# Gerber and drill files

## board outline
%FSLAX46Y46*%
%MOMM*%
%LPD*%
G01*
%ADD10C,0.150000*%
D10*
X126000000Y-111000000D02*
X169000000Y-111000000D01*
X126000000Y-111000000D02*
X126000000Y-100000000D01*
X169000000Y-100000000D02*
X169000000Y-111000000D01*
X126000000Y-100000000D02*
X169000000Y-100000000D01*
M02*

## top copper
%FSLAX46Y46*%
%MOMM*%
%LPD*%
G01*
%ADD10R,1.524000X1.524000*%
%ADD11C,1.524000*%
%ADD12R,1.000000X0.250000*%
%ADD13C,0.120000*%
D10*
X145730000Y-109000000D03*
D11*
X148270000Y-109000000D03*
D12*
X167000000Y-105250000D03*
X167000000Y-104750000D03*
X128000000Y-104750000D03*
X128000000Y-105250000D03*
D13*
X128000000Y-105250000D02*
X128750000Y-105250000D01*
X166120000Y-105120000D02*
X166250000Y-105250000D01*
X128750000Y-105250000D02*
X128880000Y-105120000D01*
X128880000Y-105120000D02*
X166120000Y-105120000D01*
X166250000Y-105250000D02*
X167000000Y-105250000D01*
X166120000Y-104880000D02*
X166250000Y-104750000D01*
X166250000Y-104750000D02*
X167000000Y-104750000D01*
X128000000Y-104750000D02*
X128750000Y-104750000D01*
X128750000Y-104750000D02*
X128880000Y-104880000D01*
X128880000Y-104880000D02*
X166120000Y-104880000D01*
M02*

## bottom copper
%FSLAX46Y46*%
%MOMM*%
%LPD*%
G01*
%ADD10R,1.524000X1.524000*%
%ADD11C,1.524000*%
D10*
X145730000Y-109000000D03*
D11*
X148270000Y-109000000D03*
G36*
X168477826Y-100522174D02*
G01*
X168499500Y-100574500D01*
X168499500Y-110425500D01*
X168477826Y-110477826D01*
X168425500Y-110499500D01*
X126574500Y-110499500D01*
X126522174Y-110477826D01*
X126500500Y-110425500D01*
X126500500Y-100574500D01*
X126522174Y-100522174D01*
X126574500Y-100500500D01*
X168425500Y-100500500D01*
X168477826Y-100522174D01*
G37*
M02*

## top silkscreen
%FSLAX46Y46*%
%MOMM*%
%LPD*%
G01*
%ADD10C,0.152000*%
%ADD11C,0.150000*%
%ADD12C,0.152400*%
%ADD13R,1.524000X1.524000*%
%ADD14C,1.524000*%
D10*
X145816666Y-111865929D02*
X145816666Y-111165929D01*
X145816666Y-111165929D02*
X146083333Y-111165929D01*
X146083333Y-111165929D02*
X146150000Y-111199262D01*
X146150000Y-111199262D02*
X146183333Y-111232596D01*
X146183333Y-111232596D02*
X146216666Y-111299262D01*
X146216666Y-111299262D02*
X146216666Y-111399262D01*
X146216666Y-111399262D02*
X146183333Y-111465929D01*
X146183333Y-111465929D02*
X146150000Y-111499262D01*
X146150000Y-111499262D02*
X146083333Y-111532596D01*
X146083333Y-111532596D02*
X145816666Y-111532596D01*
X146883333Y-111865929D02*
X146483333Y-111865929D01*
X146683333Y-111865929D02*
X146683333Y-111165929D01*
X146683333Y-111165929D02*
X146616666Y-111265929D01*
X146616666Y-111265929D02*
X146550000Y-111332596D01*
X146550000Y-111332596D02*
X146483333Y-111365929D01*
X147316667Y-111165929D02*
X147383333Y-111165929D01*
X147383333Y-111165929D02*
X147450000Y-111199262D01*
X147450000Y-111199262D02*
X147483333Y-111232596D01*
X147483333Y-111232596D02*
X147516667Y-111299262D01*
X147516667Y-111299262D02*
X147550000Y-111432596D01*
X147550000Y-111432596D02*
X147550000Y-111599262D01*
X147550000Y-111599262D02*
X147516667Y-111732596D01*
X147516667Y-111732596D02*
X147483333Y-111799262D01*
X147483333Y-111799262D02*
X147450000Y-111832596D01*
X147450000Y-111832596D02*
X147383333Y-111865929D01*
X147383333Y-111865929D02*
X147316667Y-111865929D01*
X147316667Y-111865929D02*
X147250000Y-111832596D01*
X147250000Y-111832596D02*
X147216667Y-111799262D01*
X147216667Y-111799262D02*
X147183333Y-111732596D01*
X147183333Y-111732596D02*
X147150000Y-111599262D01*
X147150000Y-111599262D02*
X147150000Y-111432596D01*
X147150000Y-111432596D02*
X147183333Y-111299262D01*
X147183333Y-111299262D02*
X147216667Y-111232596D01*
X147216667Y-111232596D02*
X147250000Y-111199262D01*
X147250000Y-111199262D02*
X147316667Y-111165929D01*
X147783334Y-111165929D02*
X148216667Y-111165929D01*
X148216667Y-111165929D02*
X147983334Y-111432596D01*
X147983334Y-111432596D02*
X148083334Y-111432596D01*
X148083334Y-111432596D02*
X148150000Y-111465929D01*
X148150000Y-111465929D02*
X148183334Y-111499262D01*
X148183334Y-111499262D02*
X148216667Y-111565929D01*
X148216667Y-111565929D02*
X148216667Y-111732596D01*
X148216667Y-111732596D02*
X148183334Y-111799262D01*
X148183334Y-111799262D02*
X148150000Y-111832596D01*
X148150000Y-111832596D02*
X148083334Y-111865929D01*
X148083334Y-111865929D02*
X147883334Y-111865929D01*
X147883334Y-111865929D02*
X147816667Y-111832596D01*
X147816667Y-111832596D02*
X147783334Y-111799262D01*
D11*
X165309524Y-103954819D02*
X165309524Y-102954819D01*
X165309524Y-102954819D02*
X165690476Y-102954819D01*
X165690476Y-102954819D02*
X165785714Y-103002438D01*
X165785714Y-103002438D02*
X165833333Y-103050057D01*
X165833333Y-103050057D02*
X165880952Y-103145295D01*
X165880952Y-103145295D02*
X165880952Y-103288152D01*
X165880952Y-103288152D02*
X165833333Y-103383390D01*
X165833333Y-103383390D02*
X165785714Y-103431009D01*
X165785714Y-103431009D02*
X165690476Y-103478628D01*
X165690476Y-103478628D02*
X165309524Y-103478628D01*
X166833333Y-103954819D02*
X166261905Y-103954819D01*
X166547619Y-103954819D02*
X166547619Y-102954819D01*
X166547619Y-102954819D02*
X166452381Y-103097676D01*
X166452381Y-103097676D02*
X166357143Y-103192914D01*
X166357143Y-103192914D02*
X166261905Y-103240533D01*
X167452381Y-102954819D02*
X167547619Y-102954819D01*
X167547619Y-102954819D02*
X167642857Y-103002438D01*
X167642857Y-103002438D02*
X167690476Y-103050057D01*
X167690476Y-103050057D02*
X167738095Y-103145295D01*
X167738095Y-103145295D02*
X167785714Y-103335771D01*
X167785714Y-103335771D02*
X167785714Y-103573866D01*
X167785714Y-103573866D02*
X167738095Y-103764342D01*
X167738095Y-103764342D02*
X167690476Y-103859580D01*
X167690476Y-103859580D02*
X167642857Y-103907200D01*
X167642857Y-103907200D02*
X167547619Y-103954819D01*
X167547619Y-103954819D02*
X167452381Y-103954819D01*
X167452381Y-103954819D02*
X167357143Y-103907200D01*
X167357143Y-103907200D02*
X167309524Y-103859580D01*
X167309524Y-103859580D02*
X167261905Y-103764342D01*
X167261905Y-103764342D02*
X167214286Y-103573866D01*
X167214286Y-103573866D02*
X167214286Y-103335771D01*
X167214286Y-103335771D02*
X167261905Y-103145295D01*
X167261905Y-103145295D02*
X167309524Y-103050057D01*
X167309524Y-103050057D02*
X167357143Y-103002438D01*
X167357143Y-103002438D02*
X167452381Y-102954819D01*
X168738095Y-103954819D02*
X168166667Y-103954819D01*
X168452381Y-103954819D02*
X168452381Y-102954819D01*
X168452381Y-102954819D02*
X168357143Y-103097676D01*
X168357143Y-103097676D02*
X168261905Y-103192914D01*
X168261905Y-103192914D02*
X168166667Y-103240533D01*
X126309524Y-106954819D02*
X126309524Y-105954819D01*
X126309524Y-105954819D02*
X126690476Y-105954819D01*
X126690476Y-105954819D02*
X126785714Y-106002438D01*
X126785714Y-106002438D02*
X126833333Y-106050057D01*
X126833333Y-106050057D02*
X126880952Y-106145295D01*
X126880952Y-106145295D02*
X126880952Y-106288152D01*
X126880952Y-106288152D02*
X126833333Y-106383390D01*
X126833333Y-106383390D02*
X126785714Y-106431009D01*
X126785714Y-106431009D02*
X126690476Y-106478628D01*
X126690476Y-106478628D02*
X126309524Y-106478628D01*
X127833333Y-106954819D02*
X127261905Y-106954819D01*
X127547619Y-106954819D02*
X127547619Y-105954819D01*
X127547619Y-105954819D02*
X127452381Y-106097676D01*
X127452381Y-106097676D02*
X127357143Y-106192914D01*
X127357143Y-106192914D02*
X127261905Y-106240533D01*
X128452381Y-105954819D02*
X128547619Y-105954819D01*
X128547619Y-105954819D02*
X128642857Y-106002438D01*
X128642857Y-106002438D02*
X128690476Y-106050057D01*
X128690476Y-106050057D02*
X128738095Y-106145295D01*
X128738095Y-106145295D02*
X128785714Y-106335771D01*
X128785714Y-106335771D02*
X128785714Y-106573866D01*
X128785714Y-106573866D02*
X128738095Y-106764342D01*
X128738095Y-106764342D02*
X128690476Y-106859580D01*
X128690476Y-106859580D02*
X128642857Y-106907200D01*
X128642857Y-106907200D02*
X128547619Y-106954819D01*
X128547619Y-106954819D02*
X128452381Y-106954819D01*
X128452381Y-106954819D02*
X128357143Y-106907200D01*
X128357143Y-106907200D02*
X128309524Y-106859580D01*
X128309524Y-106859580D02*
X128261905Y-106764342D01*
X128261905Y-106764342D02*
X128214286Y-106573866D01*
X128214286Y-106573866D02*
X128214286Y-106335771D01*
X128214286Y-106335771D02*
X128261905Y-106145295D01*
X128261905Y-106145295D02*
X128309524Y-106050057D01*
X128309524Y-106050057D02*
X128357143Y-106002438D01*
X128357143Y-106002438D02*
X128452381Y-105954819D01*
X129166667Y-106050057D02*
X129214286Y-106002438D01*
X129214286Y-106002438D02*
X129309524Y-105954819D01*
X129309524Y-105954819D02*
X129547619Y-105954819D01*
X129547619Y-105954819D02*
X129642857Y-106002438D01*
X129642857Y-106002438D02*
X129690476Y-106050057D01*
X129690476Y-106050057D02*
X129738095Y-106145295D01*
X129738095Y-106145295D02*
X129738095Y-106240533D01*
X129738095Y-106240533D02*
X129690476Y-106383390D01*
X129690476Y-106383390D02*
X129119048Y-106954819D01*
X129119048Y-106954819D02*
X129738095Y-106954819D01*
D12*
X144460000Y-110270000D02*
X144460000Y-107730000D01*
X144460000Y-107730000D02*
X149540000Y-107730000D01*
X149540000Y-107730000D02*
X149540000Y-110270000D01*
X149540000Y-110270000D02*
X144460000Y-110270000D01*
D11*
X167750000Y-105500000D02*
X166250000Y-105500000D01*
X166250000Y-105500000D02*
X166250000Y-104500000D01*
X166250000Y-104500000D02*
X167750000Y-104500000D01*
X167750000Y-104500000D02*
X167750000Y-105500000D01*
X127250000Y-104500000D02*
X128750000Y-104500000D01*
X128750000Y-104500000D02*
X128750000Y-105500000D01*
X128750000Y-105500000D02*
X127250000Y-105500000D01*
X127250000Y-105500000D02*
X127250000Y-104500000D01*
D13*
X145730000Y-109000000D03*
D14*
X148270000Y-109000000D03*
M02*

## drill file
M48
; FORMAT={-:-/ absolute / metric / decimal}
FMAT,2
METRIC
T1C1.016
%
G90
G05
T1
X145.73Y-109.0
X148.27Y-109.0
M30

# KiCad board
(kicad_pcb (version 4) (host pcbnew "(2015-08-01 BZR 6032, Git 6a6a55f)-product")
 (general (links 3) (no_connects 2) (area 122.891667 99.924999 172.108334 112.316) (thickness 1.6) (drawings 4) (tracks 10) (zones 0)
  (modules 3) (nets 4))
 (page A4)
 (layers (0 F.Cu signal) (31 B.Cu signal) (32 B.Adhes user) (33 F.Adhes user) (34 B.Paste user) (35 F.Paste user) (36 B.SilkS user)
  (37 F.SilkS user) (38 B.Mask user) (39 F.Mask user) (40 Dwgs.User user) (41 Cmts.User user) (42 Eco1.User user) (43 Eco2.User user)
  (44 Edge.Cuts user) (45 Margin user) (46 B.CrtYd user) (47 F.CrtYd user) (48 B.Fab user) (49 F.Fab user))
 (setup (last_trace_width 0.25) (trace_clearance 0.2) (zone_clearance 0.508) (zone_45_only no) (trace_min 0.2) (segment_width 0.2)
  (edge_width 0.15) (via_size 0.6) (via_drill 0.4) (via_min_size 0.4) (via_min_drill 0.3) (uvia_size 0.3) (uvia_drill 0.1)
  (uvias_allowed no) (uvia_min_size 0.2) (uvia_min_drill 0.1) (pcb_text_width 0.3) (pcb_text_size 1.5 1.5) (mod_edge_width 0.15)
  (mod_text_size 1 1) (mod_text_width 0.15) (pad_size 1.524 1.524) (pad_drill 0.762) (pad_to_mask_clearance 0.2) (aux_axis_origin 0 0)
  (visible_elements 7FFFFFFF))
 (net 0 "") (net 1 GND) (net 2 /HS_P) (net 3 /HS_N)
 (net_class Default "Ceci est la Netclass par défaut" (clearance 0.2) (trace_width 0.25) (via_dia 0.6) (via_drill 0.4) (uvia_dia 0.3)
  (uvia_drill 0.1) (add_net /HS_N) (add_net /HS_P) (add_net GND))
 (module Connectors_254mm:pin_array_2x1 (layer F.Cu) (at 147 109)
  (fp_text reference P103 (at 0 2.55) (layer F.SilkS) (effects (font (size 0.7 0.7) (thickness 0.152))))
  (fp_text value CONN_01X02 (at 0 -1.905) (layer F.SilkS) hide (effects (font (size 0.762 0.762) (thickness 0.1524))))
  (fp_line (start -2.54 1.27) (end -2.54 -1.27) (layer F.SilkS) (width 0.1524))
  (fp_line (start -2.54 -1.27) (end 2.54 -1.27) (layer F.SilkS) (width 0.1524))
  (fp_line (start 2.54 -1.27) (end 2.54 1.27) (layer F.SilkS) (width 0.1524))
  (fp_line (start 2.54 1.27) (end -2.54 1.27) (layer F.SilkS) (width 0.1524))
  (pad 1 thru_hole rect (at -1.27 0) (size 1.524 1.524) (drill 1.016) (layers *.Cu *.Mask F.SilkS) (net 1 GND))
  (pad 2 thru_hole circle (at 1.27 0) (size 1.524 1.524) (drill 1.016) (layers *.Cu *.Mask F.SilkS) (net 1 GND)))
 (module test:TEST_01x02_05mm (layer F.Cu) (at 167 105 180)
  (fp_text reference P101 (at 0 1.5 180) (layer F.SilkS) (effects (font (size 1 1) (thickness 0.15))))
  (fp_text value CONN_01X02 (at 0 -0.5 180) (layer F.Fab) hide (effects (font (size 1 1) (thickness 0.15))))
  (fp_line (start -0.75 -0.5) (end 0.75 -0.5) (layer F.SilkS) (width 0.15))
  (fp_line (start 0.75 -0.5) (end 0.75 0.5) (layer F.SilkS) (width 0.15))
  (fp_line (start 0.75 0.5) (end -0.75 0.5) (layer F.SilkS) (width 0.15))
  (fp_line (start -0.75 0.5) (end -0.75 -0.5) (layer F.SilkS) (width 0.15))
  (pad 1 smd rect (at 0 -0.25 180) (size 1 0.25) (layers F.Cu F.Paste F.Mask) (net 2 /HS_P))
  (pad 2 smd rect (at 0 0.25 180) (size 1 0.25) (layers F.Cu F.Paste F.Mask) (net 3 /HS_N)))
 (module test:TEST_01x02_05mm (layer F.Cu) (at 128 105)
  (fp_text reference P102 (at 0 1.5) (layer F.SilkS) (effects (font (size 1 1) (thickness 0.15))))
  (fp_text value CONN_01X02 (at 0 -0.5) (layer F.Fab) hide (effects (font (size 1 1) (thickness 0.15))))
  (fp_line (start -0.75 -0.5) (end 0.75 -0.5) (layer F.SilkS) (width 0.15))
  (fp_line (start 0.75 -0.5) (end 0.75 0.5) (layer F.SilkS) (width 0.15))
  (fp_line (start 0.75 0.5) (end -0.75 0.5) (layer F.SilkS) (width 0.15))
  (fp_line (start -0.75 0.5) (end -0.75 -0.5) (layer F.SilkS) (width 0.15))
  (pad 1 smd rect (at 0 -0.25) (size 1 0.25) (layers F.Cu F.Paste F.Mask) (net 3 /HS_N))
  (pad 2 smd rect (at 0 0.25) (size 1 0.25) (layers F.Cu F.Paste F.Mask) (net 2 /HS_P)))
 (gr_line (start 126 111) (end 169 111) (layer Edge.Cuts) (width 0.15))
 (gr_line (start 126 111) (end 126 100) (layer Edge.Cuts) (width 0.15))
 (gr_line (start 169 100) (end 169 111) (layer Edge.Cuts) (width 0.15))
 (gr_line (start 126 100) (end 169 100) (layer Edge.Cuts) (width 0.15))
 (segment (start 128 105.25) (end 128.75 105.25) (width 0.12) (layer F.Cu) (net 2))
 (segment (start 166.12 105.12) (end 166.25 105.25) (width 0.12) (layer F.Cu) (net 2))
 (segment (start 128.75 105.25) (end 128.88 105.12) (width 0.12) (layer F.Cu) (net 2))
 (segment (start 128.88 105.12) (end 166.12 105.12) (width 0.12) (layer F.Cu) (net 2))
 (segment (start 166.25 105.25) (end 167 105.25) (width 0.12) (layer F.Cu) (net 2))
 (segment (start 166.12 104.88) (end 166.25 104.75) (width 0.12) (layer F.Cu) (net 3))
 (segment (start 166.25 104.75) (end 167 104.75) (width 0.12) (layer F.Cu) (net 3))
 (segment (start 128 104.75) (end 128.75 104.75) (width 0.12) (layer F.Cu) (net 3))
 (segment (start 128.75 104.75) (end 128.88 104.88) (width 0.12) (layer F.Cu) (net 3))
 (segment (start 128.88 104.88) (end 166.12 104.88) (width 0.12) (layer F.Cu) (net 3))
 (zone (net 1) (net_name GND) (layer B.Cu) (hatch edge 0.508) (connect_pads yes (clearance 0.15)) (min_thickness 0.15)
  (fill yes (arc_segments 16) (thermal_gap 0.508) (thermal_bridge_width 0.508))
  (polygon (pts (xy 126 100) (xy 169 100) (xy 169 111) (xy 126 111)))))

